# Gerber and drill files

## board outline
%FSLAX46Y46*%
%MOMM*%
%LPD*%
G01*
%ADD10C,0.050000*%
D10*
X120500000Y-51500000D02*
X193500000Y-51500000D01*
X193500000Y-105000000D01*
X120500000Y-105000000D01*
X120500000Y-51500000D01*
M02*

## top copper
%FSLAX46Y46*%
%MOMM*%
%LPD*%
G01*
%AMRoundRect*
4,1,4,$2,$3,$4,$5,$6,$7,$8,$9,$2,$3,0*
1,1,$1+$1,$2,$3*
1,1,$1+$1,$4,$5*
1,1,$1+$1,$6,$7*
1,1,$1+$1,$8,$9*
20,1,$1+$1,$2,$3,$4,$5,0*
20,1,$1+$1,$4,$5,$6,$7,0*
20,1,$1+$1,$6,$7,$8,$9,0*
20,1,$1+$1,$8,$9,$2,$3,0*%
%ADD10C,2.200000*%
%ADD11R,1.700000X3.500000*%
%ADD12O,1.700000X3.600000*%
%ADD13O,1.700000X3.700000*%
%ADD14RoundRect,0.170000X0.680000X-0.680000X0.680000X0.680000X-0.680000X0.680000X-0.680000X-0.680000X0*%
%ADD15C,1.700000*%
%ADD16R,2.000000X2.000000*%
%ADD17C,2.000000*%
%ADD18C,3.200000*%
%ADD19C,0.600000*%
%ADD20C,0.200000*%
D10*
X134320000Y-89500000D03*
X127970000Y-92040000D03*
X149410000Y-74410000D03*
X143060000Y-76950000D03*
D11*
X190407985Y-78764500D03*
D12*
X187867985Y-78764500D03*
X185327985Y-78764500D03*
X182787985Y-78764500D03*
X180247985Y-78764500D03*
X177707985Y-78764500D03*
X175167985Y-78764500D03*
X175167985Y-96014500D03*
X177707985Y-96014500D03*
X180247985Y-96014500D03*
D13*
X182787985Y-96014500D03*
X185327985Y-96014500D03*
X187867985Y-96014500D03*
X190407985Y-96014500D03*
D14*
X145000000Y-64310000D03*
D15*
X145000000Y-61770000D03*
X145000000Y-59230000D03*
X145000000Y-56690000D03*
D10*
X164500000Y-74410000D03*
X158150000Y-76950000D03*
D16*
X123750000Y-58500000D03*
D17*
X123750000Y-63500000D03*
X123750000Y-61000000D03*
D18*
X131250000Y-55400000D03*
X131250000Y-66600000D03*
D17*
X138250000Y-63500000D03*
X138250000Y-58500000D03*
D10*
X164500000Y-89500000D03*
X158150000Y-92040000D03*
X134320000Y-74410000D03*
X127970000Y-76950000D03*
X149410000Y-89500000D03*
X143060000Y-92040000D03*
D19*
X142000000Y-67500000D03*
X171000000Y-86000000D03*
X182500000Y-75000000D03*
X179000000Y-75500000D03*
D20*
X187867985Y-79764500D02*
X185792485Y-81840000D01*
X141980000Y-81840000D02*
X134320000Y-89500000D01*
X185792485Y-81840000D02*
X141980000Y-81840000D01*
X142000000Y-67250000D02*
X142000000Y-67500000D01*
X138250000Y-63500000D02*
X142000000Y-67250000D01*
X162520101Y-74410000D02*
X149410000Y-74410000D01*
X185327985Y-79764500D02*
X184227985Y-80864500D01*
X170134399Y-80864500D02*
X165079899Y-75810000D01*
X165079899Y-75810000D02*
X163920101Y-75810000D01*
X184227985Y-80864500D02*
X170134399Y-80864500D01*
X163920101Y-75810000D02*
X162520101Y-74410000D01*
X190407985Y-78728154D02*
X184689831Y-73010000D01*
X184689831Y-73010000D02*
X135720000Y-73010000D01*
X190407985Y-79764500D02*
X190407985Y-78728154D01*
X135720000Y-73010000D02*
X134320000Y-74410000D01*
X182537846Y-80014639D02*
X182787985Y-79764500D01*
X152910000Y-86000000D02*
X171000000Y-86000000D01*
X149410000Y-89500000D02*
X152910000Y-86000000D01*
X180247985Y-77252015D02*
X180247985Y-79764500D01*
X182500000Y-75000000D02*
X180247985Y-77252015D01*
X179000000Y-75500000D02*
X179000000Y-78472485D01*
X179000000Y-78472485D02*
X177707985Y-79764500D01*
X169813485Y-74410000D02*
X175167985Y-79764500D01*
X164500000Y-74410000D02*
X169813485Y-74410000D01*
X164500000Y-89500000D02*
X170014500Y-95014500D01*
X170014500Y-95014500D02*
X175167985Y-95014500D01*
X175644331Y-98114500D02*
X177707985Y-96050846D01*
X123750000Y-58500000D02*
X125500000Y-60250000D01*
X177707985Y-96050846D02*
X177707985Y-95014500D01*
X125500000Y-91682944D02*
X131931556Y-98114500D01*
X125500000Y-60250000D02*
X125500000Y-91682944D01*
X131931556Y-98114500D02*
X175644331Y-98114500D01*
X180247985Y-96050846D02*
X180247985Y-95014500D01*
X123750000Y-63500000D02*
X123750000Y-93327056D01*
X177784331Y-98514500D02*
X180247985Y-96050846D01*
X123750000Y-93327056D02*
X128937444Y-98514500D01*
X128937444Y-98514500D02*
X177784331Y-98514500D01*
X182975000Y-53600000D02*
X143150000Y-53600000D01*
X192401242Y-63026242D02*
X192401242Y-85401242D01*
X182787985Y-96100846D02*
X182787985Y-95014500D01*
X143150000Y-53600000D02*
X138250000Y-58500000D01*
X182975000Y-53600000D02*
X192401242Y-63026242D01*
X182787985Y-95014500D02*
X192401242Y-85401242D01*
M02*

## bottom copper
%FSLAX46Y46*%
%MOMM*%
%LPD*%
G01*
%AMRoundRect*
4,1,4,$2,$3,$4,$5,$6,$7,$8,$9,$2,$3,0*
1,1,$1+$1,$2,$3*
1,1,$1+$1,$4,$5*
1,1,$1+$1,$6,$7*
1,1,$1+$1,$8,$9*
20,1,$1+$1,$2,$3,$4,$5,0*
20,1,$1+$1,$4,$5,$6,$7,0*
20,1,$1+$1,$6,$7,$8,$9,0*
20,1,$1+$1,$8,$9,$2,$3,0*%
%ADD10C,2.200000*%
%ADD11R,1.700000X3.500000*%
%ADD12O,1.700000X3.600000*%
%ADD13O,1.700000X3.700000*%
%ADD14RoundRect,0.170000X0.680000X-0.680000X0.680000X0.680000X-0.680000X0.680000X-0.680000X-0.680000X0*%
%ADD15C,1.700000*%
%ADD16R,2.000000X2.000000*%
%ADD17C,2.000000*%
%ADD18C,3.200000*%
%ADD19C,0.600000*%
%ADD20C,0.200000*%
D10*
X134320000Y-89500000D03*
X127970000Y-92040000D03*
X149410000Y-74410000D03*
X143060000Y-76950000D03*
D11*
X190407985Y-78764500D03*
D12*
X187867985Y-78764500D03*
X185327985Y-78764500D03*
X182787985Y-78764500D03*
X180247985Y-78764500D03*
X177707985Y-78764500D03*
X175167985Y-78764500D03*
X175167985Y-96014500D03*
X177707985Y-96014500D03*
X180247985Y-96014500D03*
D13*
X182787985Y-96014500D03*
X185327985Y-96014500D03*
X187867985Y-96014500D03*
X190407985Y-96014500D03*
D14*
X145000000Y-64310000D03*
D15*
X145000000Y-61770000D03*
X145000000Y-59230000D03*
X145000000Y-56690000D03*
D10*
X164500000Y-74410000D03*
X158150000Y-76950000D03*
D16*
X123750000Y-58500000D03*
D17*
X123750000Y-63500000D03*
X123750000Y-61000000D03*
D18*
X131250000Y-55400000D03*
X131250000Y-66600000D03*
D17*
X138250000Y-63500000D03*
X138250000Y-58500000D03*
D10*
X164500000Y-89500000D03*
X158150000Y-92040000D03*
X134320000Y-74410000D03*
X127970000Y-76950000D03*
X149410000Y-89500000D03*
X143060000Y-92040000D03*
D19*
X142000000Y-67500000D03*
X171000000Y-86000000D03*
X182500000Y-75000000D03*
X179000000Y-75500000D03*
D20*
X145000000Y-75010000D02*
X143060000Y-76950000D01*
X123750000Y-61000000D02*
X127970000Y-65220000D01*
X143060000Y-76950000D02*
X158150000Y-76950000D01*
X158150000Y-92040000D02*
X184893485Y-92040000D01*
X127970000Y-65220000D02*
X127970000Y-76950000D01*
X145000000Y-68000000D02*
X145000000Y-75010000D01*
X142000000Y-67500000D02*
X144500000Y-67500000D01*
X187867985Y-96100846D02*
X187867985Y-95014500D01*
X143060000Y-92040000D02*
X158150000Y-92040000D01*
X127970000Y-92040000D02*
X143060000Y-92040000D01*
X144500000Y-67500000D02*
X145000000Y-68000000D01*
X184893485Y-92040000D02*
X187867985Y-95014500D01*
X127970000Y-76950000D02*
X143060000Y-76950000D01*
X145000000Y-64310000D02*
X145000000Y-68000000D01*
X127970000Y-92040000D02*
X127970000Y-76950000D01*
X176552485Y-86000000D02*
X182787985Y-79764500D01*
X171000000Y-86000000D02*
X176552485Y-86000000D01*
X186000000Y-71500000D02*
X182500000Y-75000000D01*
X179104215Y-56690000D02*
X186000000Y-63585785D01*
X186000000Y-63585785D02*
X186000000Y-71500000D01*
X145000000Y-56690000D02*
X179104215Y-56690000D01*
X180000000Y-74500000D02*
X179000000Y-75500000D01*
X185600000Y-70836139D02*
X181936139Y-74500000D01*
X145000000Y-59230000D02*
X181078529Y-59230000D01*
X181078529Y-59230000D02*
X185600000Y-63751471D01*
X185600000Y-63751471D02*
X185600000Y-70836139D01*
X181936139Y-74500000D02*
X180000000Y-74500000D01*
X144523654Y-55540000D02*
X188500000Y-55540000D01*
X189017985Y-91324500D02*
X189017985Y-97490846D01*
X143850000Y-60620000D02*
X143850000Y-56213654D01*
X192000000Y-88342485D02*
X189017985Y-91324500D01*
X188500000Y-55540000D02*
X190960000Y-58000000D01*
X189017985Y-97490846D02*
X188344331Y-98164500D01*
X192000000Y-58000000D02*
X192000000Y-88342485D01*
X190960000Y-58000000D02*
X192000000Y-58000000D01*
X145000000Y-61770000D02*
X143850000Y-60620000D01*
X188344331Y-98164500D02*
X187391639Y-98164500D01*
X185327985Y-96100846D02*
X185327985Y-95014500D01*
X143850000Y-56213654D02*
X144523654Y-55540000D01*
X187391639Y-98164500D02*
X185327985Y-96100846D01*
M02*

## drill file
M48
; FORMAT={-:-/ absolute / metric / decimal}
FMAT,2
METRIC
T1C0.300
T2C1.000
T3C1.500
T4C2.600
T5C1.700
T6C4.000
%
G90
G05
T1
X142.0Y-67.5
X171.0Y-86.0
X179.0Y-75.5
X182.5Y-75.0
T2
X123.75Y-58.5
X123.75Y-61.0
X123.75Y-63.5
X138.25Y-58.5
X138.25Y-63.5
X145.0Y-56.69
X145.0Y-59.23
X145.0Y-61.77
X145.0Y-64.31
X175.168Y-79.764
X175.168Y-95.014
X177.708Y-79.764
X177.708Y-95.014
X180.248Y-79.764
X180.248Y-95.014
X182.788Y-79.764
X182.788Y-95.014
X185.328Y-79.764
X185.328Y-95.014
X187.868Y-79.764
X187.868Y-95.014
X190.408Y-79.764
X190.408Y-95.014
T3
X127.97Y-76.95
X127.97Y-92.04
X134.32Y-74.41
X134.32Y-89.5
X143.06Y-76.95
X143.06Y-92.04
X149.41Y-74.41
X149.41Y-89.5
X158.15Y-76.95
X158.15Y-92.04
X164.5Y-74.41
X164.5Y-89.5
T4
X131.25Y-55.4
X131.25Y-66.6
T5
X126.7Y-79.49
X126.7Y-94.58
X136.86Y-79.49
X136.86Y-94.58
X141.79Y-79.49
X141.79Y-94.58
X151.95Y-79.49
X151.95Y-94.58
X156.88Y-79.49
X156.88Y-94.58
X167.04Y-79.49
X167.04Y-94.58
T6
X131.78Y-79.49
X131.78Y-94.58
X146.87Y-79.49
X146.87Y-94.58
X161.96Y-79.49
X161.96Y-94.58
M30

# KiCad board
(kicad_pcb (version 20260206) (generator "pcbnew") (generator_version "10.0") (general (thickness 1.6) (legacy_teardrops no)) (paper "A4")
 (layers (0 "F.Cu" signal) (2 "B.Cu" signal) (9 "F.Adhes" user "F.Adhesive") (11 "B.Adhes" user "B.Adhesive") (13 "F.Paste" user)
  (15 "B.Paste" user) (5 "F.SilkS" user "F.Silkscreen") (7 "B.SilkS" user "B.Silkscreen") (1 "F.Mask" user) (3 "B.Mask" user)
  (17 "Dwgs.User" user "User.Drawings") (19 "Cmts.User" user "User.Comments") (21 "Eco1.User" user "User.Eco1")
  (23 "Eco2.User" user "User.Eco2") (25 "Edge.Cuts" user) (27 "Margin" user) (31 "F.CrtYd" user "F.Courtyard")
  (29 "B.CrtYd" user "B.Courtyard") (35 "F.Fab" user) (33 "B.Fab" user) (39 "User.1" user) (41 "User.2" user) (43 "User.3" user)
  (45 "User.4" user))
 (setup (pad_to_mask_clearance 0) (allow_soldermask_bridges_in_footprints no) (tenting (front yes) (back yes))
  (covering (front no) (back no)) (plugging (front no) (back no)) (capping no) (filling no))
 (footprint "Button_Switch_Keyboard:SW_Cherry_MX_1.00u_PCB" (layer "F.Cu") (at 134.32 89.5)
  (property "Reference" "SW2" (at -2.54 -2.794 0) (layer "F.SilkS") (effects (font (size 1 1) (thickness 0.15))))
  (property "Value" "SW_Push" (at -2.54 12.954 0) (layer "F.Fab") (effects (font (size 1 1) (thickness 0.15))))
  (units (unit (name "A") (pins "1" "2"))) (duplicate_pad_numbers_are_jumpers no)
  (pad "" np_thru_hole circle (at -7.62 5.08) (size 1.7 1.7) (drill 1.7) (layers "*.Cu" "*.Mask"))
  (pad "" np_thru_hole circle (at -2.54 5.08) (size 4 4) (drill 4) (layers "*.Cu" "*.Mask"))
  (pad "" np_thru_hole circle (at 2.54 5.08) (size 1.7 1.7) (drill 1.7) (layers "*.Cu" "*.Mask"))
  (pad "1" thru_hole circle (at 0 0) (size 2.2 2.2) (drill 1.5) (layers "*.Cu" "*.Mask") (remove_unused_layers no)
   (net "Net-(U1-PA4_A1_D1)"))
  (pad "2" thru_hole circle (at -6.35 2.54) (size 2.2 2.2) (drill 1.5) (layers "*.Cu" "*.Mask") (remove_unused_layers no) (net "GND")))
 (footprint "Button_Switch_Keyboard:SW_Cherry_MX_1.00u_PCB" (layer "F.Cu") (at 149.41 74.41)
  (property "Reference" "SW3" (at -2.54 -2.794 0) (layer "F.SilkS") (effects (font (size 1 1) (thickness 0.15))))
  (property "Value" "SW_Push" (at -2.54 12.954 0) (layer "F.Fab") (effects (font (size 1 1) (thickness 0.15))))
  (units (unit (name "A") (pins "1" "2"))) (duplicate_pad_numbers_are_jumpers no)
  (pad "" np_thru_hole circle (at -7.62 5.08) (size 1.7 1.7) (drill 1.7) (layers "*.Cu" "*.Mask"))
  (pad "" np_thru_hole circle (at -2.54 5.08) (size 4 4) (drill 4) (layers "*.Cu" "*.Mask"))
  (pad "" np_thru_hole circle (at 2.54 5.08) (size 1.7 1.7) (drill 1.7) (layers "*.Cu" "*.Mask"))
  (pad "1" thru_hole circle (at 0 0) (size 2.2 2.2) (drill 1.5) (layers "*.Cu" "*.Mask") (remove_unused_layers no)
   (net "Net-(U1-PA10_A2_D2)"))
  (pad "2" thru_hole circle (at -6.35 2.54) (size 2.2 2.2) (drill 1.5) (layers "*.Cu" "*.Mask") (remove_unused_layers no) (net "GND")))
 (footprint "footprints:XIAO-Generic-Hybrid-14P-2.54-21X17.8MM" (layer "F.Cu") (at 182.787985 87.3895 -90)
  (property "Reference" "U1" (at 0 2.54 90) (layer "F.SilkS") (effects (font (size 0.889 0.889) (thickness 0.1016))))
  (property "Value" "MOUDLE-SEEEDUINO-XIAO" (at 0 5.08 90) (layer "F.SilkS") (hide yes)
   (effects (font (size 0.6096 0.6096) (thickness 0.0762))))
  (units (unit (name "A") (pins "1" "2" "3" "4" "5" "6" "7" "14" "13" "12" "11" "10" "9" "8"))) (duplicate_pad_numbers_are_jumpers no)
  (pad "1" thru_hole rect (at -7.625 -7.62 270) (size 3.5 1.7) (drill 1 (offset -1 0)) (layers "*.Cu" "*.Mask") (remove_unused_layers no)
   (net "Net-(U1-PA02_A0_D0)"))
  (pad "2" thru_hole oval (at -7.625 -5.08 270) (size 3.6 1.7) (drill 1 (offset -1 0)) (layers "*.Cu" "*.Mask") (remove_unused_layers no)
   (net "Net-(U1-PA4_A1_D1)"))
  (pad "3" thru_hole oval (at -7.625 -2.54 270) (size 3.6 1.7) (drill 1 (offset -1 0)) (layers "*.Cu" "*.Mask") (remove_unused_layers no)
   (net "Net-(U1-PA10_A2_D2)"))
  (pad "4" thru_hole oval (at -7.625 0 270) (size 3.6 1.7) (drill 1 (offset -1 0)) (layers "*.Cu" "*.Mask") (remove_unused_layers no)
   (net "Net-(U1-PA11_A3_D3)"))
  (pad "5" thru_hole oval (at -7.625 2.54 270) (size 3.6 1.7) (drill 1 (offset -1 0)) (layers "*.Cu" "*.Mask") (remove_unused_layers no)
   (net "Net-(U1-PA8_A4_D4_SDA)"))
  (pad "6" thru_hole oval (at -7.625 5.08 90) (size 3.6 1.7) (drill 1 (offset 1 0)) (layers "*.Cu" "*.Mask") (remove_unused_layers no)
   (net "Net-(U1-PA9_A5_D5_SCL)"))
  (pad "7" thru_hole oval (at -7.625 7.62 270) (size 3.6 1.7) (drill 1 (offset -1 0)) (layers "*.Cu" "*.Mask") (remove_unused_layers no)
   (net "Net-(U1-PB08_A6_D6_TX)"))
  (pad "8" thru_hole oval (at 7.625 7.62 270) (size 3.6 1.7) (drill 1 (offset 1 0)) (layers "*.Cu" "*.Mask") (remove_unused_layers no)
   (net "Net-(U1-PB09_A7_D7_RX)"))
  (pad "9" thru_hole oval (at 7.625 5.08 270) (size 3.6 1.7) (drill 1 (offset 1 0)) (layers "*.Cu" "*.Mask") (remove_unused_layers no)
   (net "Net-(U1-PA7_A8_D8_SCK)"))
  (pad "10" thru_hole oval (at 7.625 2.54 270) (size 3.6 1.7) (drill 1 (offset 1 0)) (layers "*.Cu" "*.Mask") (remove_unused_layers no)
   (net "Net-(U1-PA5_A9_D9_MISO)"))
  (pad "11" thru_hole oval (at 7.625 0 270) (size 3.7 1.7) (drill 1 (offset 1 0)) (layers "*.Cu" "*.Mask") (remove_unused_layers no)
   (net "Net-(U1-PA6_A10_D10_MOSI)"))
  (pad "12" thru_hole oval (at 7.625 -2.54 270) (size 3.7 1.7) (drill 1 (offset 1 0)) (layers "*.Cu" "*.Mask") (remove_unused_layers no)
   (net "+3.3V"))
  (pad "13" thru_hole oval (at 7.625 -5.08 270) (size 3.7 1.7) (drill 1 (offset 1 0)) (layers "*.Cu" "*.Mask") (remove_unused_layers no)
   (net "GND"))
  (pad "14" thru_hole oval (at 7.625 -7.62 270) (size 3.7 1.7) (drill 1 (offset 1 0)) (layers "*.Cu" "*.Mask") (remove_unused_layers no)
   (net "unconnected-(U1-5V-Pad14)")))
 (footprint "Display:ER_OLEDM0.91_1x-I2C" (layer "F.Cu") (at 145 64.31 90)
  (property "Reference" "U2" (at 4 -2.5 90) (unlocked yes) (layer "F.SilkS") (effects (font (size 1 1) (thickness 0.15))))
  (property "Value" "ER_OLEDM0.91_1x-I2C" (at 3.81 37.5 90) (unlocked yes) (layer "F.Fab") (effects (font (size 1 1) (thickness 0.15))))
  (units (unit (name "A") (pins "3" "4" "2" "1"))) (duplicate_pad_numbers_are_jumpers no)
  (pad "1" thru_hole roundrect (at 0 0 90) (size 1.7 1.7) (drill 1) (layers "*.Cu" "*.Mask") (remove_unused_layers no)
   (roundrect_rratio 0.1) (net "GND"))
  (pad "2" thru_hole circle (at 2.54 0 90) (size 1.7 1.7) (drill 1) (layers "*.Cu" "*.Mask") (remove_unused_layers no) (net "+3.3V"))
  (pad "3" thru_hole circle (at 5.08 0 90) (size 1.7 1.7) (drill 1) (layers "*.Cu" "*.Mask") (remove_unused_layers no)
   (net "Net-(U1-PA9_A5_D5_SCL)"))
  (pad "4" thru_hole circle (at 7.62 0 90) (size 1.7 1.7) (drill 1) (layers "*.Cu" "*.Mask") (remove_unused_layers no)
   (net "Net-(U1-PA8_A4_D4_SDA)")))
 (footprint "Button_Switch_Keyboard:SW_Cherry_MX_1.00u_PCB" (layer "F.Cu") (at 164.5 74.41)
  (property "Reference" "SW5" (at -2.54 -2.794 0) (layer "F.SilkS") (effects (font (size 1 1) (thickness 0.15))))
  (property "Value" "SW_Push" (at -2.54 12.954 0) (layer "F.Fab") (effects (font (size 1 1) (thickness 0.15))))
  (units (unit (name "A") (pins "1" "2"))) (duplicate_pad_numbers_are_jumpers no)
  (pad "" np_thru_hole circle (at -7.62 5.08) (size 1.7 1.7) (drill 1.7) (layers "*.Cu" "*.Mask"))
  (pad "" np_thru_hole circle (at -2.54 5.08) (size 4 4) (drill 4) (layers "*.Cu" "*.Mask"))
  (pad "" np_thru_hole circle (at 2.54 5.08) (size 1.7 1.7) (drill 1.7) (layers "*.Cu" "*.Mask"))
  (pad "1" thru_hole circle (at 0 0) (size 2.2 2.2) (drill 1.5) (layers "*.Cu" "*.Mask") (remove_unused_layers no)
   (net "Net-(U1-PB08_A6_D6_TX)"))
  (pad "2" thru_hole circle (at -6.35 2.54) (size 2.2 2.2) (drill 1.5) (layers "*.Cu" "*.Mask") (remove_unused_layers no) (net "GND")))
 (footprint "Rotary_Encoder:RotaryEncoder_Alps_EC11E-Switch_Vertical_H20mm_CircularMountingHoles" (layer "F.Cu") (at 123.75 58.5)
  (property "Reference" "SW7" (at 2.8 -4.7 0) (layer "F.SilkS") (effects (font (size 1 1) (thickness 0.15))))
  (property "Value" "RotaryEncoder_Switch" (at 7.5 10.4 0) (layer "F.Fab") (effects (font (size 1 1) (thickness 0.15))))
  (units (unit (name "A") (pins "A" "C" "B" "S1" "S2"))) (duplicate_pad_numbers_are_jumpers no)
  (pad "A" thru_hole rect (at 0 0) (size 2 2) (drill 1) (layers "*.Cu" "*.Mask") (remove_unused_layers no) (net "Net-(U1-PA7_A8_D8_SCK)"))
  (pad "B" thru_hole circle (at 0 5) (size 2 2) (drill 1) (layers "*.Cu" "*.Mask") (remove_unused_layers no) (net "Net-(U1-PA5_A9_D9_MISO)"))
  (pad "C" thru_hole circle (at 0 2.5) (size 2 2) (drill 1) (layers "*.Cu" "*.Mask") (remove_unused_layers no) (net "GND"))
  (pad "MP" thru_hole circle (at 7.5 -3.1) (size 3.2 3.2) (drill 2.6) (layers "*.Cu" "*.Mask") (remove_unused_layers no))
  (pad "MP" thru_hole circle (at 7.5 8.1) (size 3.2 3.2) (drill 2.6) (layers "*.Cu" "*.Mask") (remove_unused_layers no))
  (pad "S1" thru_hole circle (at 14.5 5) (size 2 2) (drill 1) (layers "*.Cu" "*.Mask") (remove_unused_layers no) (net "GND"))
  (pad "S2" thru_hole circle (at 14.5 0) (size 2 2) (drill 1) (layers "*.Cu" "*.Mask") (remove_unused_layers no)
   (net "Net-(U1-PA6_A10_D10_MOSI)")))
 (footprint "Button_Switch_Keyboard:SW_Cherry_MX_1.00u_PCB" (layer "F.Cu") (at 164.5 89.5)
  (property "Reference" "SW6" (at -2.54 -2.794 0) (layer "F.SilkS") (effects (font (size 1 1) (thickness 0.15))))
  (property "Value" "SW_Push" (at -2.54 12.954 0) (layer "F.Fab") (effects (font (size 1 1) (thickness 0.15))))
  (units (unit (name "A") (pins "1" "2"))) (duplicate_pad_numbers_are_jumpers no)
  (pad "" np_thru_hole circle (at -7.62 5.08) (size 1.7 1.7) (drill 1.7) (layers "*.Cu" "*.Mask"))
  (pad "" np_thru_hole circle (at -2.54 5.08) (size 4 4) (drill 4) (layers "*.Cu" "*.Mask"))
  (pad "" np_thru_hole circle (at 2.54 5.08) (size 1.7 1.7) (drill 1.7) (layers "*.Cu" "*.Mask"))
  (pad "1" thru_hole circle (at 0 0) (size 2.2 2.2) (drill 1.5) (layers "*.Cu" "*.Mask") (remove_unused_layers no)
   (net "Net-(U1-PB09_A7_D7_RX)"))
  (pad "2" thru_hole circle (at -6.35 2.54) (size 2.2 2.2) (drill 1.5) (layers "*.Cu" "*.Mask") (remove_unused_layers no) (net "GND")))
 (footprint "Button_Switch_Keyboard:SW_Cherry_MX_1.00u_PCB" (layer "F.Cu") (at 134.32 74.41)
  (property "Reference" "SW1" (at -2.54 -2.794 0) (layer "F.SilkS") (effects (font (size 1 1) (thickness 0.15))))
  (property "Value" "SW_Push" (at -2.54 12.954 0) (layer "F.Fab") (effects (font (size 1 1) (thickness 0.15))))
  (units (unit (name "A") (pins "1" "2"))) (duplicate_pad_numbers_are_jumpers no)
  (pad "" np_thru_hole circle (at -7.62 5.08) (size 1.7 1.7) (drill 1.7) (layers "*.Cu" "*.Mask"))
  (pad "" np_thru_hole circle (at -2.54 5.08) (size 4 4) (drill 4) (layers "*.Cu" "*.Mask"))
  (pad "" np_thru_hole circle (at 2.54 5.08) (size 1.7 1.7) (drill 1.7) (layers "*.Cu" "*.Mask"))
  (pad "1" thru_hole circle (at 0 0) (size 2.2 2.2) (drill 1.5) (layers "*.Cu" "*.Mask") (remove_unused_layers no)
   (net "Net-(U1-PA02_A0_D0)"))
  (pad "2" thru_hole circle (at -6.35 2.54) (size 2.2 2.2) (drill 1.5) (layers "*.Cu" "*.Mask") (remove_unused_layers no) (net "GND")))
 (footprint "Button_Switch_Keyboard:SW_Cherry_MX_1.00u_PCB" (layer "F.Cu") (at 149.41 89.5)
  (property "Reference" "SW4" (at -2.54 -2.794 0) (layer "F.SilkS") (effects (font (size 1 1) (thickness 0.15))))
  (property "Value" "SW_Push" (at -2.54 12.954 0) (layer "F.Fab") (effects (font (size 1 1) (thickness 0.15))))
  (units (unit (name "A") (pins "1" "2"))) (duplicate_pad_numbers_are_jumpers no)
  (pad "" np_thru_hole circle (at -7.62 5.08) (size 1.7 1.7) (drill 1.7) (layers "*.Cu" "*.Mask"))
  (pad "" np_thru_hole circle (at -2.54 5.08) (size 4 4) (drill 4) (layers "*.Cu" "*.Mask"))
  (pad "" np_thru_hole circle (at 2.54 5.08) (size 1.7 1.7) (drill 1.7) (layers "*.Cu" "*.Mask"))
  (pad "1" thru_hole circle (at 0 0) (size 2.2 2.2) (drill 1.5) (layers "*.Cu" "*.Mask") (remove_unused_layers no)
   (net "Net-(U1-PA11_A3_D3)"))
  (pad "2" thru_hole circle (at -6.35 2.54) (size 2.2 2.2) (drill 1.5) (layers "*.Cu" "*.Mask") (remove_unused_layers no) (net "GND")))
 (gr_rect (start 120.5 51.5) (end 193.5 105) (stroke (width 0.05) (type default)) (fill no) (layer "Edge.Cuts"))
 (segment (start 187.867985 79.7645) (end 185.792485 81.84) (width 0.2) (layer "F.Cu") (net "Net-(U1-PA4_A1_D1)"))
 (segment (start 141.98 81.84) (end 134.32 89.5) (width 0.2) (layer "F.Cu") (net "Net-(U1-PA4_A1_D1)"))
 (segment (start 185.792485 81.84) (end 141.98 81.84) (width 0.2) (layer "F.Cu") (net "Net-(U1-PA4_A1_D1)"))
 (segment (start 142 67.25) (end 142 67.5) (width 0.2) (layer "F.Cu") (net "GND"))
 (segment (start 138.25 63.5) (end 142 67.25) (width 0.2) (layer "F.Cu") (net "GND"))
 (via (at 142 67.5) (size 0.6) (drill 0.3) (layers "F.Cu" "B.Cu") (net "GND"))
 (segment (start 145 75.01) (end 143.06 76.95) (width 0.2) (layer "B.Cu") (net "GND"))
 (segment (start 123.75 61) (end 127.97 65.22) (width 0.2) (layer "B.Cu") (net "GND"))
 (segment (start 143.06 76.95) (end 158.15 76.95) (width 0.2) (layer "B.Cu") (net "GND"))
 (segment (start 158.15 92.04) (end 184.893485 92.04) (width 0.2) (layer "B.Cu") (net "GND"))
 (segment (start 127.97 65.22) (end 127.97 76.95) (width 0.2) (layer "B.Cu") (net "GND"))
 (segment (start 145 68) (end 145 75.01) (width 0.2) (layer "B.Cu") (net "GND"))
 (segment (start 142 67.5) (end 144.5 67.5) (width 0.2) (layer "B.Cu") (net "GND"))
 (segment (start 187.867985 96.100846) (end 187.867985 95.0145) (width 0.2) (layer "B.Cu") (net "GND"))
 (segment (start 143.06 92.04) (end 158.15 92.04) (width 0.2) (layer "B.Cu") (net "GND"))
 (segment (start 127.97 92.04) (end 143.06 92.04) (width 0.2) (layer "B.Cu") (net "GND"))
 (segment (start 144.5 67.5) (end 145 68) (width 0.2) (layer "B.Cu") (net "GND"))
 (segment (start 184.893485 92.04) (end 187.867985 95.0145) (width 0.2) (layer "B.Cu") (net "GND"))
 (segment (start 127.97 76.95) (end 143.06 76.95) (width 0.2) (layer "B.Cu") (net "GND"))
 (segment (start 145 64.31) (end 145 68) (width 0.2) (layer "B.Cu") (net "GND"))
 (segment (start 127.97 92.04) (end 127.97 76.95) (width 0.2) (layer "B.Cu") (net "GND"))
 (segment (start 162.520101 74.41) (end 149.41 74.41) (width 0.2) (layer "F.Cu") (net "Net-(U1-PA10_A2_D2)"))
 (segment (start 185.327985 79.7645) (end 184.227985 80.8645) (width 0.2) (layer "F.Cu") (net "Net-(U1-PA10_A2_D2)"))
 (segment (start 170.134399 80.8645) (end 165.079899 75.81) (width 0.2) (layer "F.Cu") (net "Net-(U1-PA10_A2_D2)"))
 (segment (start 165.079899 75.81) (end 163.920101 75.81) (width 0.2) (layer "F.Cu") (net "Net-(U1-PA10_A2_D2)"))
 (segment (start 184.227985 80.8645) (end 170.134399 80.8645) (width 0.2) (layer "F.Cu") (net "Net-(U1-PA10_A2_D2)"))
 (segment (start 163.920101 75.81) (end 162.520101 74.41) (width 0.2) (layer "F.Cu") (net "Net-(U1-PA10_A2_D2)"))
 (segment (start 190.407985 78.728154) (end 184.689831 73.01) (width 0.2) (layer "F.Cu") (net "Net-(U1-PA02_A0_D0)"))
 (segment (start 184.689831 73.01) (end 135.72 73.01) (width 0.2) (layer "F.Cu") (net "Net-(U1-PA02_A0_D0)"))
 (segment (start 190.407985 79.7645) (end 190.407985 78.728154) (width 0.2) (layer "F.Cu") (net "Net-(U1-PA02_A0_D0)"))
 (segment (start 135.72 73.01) (end 134.32 74.41) (width 0.2) (layer "F.Cu") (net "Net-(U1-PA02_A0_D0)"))
 (segment (start 182.537846 80.014639) (end 182.787985 79.7645) (width 0.2) (layer "F.Cu") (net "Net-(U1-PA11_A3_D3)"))
 (segment (start 152.91 86) (end 171 86) (width 0.2) (layer "F.Cu") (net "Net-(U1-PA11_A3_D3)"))
 (segment (start 149.41 89.5) (end 152.91 86) (width 0.2) (layer "F.Cu") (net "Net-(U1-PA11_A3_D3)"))
 (via (at 171 86) (size 0.6) (drill 0.3) (layers "F.Cu" "B.Cu") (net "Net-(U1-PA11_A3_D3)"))
 (segment (start 176.552485 86) (end 182.787985 79.7645) (width 0.2) (layer "B.Cu") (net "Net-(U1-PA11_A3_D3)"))
 (segment (start 171 86) (end 176.552485 86) (width 0.2) (layer "B.Cu") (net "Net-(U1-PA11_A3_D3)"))
 (segment (start 180.247985 77.252015) (end 180.247985 79.7645) (width 0.2) (layer "F.Cu") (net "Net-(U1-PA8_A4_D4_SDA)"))
 (segment (start 182.5 75) (end 180.247985 77.252015) (width 0.2) (layer "F.Cu") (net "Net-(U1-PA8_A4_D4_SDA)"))
 (via (at 182.5 75) (size 0.6) (drill 0.3) (layers "F.Cu" "B.Cu") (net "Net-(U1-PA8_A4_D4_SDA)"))
 (segment (start 186 71.5) (end 182.5 75) (width 0.2) (layer "B.Cu") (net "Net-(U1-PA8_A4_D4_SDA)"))
 (segment (start 179.104215 56.69) (end 186 63.585785) (width 0.2) (layer "B.Cu") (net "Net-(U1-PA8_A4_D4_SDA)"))
 (segment (start 186 63.585785) (end 186 71.5) (width 0.2) (layer "B.Cu") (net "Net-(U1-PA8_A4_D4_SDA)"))
 (segment (start 145 56.69) (end 179.104215 56.69) (width 0.2) (layer "B.Cu") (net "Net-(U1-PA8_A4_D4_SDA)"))
 (segment (start 179 75.5) (end 179 78.472485) (width 0.2) (layer "F.Cu") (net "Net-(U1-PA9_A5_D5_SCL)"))
 (segment (start 179 78.472485) (end 177.707985 79.7645) (width 0.2) (layer "F.Cu") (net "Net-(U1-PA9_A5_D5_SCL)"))
 (via (at 179 75.5) (size 0.6) (drill 0.3) (layers "F.Cu" "B.Cu") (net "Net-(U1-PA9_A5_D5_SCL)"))
 (segment (start 180 74.5) (end 179 75.5) (width 0.2) (layer "B.Cu") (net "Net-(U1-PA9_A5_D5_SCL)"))
 (segment (start 185.6 70.836139) (end 181.936139 74.5) (width 0.2) (layer "B.Cu") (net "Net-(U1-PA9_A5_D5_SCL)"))
 (segment (start 145 59.23) (end 181.078529 59.23) (width 0.2) (layer "B.Cu") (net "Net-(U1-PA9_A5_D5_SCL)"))
 (segment (start 181.078529 59.23) (end 185.6 63.751471) (width 0.2) (layer "B.Cu") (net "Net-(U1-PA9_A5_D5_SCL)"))
 (segment (start 185.6 63.751471) (end 185.6 70.836139) (width 0.2) (layer "B.Cu") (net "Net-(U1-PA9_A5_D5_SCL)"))
 (segment (start 181.936139 74.5) (end 180 74.5) (width 0.2) (layer "B.Cu") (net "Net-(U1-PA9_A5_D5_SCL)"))
 (segment (start 169.813485 74.41) (end 175.167985 79.7645) (width 0.2) (layer "F.Cu") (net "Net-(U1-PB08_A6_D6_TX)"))
 (segment (start 164.5 74.41) (end 169.813485 74.41) (width 0.2) (layer "F.Cu") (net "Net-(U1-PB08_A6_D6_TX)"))
 (segment (start 164.5 89.5) (end 170.0145 95.0145) (width 0.2) (layer "F.Cu") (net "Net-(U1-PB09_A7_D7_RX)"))
 (segment (start 170.0145 95.0145) (end 175.167985 95.0145) (width 0.2) (layer "F.Cu") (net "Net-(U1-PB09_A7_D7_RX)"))
 (segment (start 175.644331 98.1145) (end 177.707985 96.050846) (width 0.2) (layer "F.Cu") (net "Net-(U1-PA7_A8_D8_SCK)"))
 (segment (start 123.75 58.5) (end 125.5 60.25) (width 0.2) (layer "F.Cu") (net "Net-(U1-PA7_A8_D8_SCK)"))
 (segment (start 177.707985 96.050846) (end 177.707985 95.0145) (width 0.2) (layer "F.Cu") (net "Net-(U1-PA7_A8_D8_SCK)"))
 (segment (start 125.5 91.682944) (end 131.931556 98.1145) (width 0.2) (layer "F.Cu") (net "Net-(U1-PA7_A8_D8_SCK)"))
 (segment (start 125.5 60.25) (end 125.5 91.682944) (width 0.2) (layer "F.Cu") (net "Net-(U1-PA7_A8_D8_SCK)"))
 (segment (start 131.931556 98.1145) (end 175.644331 98.1145) (width 0.2) (layer "F.Cu") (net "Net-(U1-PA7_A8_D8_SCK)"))
 (segment (start 180.247985 96.050846) (end 180.247985 95.0145) (width 0.2) (layer "F.Cu") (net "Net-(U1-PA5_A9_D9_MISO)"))
 (segment (start 123.75 63.5) (end 123.75 93.327056) (width 0.2) (layer "F.Cu") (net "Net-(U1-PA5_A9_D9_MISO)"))
 (segment (start 177.784331 98.5145) (end 180.247985 96.050846) (width 0.2) (layer "F.Cu") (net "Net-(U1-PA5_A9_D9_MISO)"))
 (segment (start 123.75 93.327056) (end 128.937444 98.5145) (width 0.2) (layer "F.Cu") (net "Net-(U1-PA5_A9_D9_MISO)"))
 (segment (start 128.937444 98.5145) (end 177.784331 98.5145) (width 0.2) (layer "F.Cu") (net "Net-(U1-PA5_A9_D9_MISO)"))
 (segment (start 182.975 53.6) (end 143.15 53.6) (width 0.2) (layer "F.Cu") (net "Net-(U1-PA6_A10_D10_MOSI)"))
 (segment (start 192.401242 63.026242) (end 192.401242 85.401242) (width 0.2) (layer "F.Cu") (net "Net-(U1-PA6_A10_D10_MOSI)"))
 (segment (start 182.787985 96.100846) (end 182.787985 95.0145) (width 0.2) (layer "F.Cu") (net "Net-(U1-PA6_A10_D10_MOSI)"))
 (segment (start 143.15 53.6) (end 138.25 58.5) (width 0.2) (layer "F.Cu") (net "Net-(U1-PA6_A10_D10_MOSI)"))
 (segment (start 182.975 53.6) (end 192.401242 63.026242) (width 0.2) (layer "F.Cu") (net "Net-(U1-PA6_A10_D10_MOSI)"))
 (segment (start 182.787985 95.0145) (end 192.401242 85.401242) (width 0.2) (layer "F.Cu") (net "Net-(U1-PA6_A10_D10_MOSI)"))
 (segment (start 144.523654 55.54) (end 188.5 55.54) (width 0.2) (layer "B.Cu") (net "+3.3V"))
 (segment (start 189.017985 91.3245) (end 189.017985 97.490846) (width 0.2) (layer "B.Cu") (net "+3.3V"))
 (segment (start 143.85 60.62) (end 143.85 56.213654) (width 0.2) (layer "B.Cu") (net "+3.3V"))
 (segment (start 192 88.342485) (end 189.017985 91.3245) (width 0.2) (layer "B.Cu") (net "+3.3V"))
 (segment (start 188.5 55.54) (end 190.96 58) (width 0.2) (layer "B.Cu") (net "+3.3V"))
 (segment (start 189.017985 97.490846) (end 188.344331 98.1645) (width 0.2) (layer "B.Cu") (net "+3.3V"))
 (segment (start 192 58) (end 192 88.342485) (width 0.2) (layer "B.Cu") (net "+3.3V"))
 (segment (start 190.96 58) (end 192 58) (width 0.2) (layer "B.Cu") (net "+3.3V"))
 (segment (start 145 61.77) (end 143.85 60.62) (width 0.2) (layer "B.Cu") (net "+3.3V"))
 (segment (start 188.344331 98.1645) (end 187.391639 98.1645) (width 0.2) (layer "B.Cu") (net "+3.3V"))
 (segment (start 185.327985 96.100846) (end 185.327985 95.0145) (width 0.2) (layer "B.Cu") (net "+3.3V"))
 (segment (start 143.85 56.213654) (end 144.523654 55.54) (width 0.2) (layer "B.Cu") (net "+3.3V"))
 (segment (start 187.391639 98.1645) (end 185.327985 96.100846) (width 0.2) (layer "B.Cu") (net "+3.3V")))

